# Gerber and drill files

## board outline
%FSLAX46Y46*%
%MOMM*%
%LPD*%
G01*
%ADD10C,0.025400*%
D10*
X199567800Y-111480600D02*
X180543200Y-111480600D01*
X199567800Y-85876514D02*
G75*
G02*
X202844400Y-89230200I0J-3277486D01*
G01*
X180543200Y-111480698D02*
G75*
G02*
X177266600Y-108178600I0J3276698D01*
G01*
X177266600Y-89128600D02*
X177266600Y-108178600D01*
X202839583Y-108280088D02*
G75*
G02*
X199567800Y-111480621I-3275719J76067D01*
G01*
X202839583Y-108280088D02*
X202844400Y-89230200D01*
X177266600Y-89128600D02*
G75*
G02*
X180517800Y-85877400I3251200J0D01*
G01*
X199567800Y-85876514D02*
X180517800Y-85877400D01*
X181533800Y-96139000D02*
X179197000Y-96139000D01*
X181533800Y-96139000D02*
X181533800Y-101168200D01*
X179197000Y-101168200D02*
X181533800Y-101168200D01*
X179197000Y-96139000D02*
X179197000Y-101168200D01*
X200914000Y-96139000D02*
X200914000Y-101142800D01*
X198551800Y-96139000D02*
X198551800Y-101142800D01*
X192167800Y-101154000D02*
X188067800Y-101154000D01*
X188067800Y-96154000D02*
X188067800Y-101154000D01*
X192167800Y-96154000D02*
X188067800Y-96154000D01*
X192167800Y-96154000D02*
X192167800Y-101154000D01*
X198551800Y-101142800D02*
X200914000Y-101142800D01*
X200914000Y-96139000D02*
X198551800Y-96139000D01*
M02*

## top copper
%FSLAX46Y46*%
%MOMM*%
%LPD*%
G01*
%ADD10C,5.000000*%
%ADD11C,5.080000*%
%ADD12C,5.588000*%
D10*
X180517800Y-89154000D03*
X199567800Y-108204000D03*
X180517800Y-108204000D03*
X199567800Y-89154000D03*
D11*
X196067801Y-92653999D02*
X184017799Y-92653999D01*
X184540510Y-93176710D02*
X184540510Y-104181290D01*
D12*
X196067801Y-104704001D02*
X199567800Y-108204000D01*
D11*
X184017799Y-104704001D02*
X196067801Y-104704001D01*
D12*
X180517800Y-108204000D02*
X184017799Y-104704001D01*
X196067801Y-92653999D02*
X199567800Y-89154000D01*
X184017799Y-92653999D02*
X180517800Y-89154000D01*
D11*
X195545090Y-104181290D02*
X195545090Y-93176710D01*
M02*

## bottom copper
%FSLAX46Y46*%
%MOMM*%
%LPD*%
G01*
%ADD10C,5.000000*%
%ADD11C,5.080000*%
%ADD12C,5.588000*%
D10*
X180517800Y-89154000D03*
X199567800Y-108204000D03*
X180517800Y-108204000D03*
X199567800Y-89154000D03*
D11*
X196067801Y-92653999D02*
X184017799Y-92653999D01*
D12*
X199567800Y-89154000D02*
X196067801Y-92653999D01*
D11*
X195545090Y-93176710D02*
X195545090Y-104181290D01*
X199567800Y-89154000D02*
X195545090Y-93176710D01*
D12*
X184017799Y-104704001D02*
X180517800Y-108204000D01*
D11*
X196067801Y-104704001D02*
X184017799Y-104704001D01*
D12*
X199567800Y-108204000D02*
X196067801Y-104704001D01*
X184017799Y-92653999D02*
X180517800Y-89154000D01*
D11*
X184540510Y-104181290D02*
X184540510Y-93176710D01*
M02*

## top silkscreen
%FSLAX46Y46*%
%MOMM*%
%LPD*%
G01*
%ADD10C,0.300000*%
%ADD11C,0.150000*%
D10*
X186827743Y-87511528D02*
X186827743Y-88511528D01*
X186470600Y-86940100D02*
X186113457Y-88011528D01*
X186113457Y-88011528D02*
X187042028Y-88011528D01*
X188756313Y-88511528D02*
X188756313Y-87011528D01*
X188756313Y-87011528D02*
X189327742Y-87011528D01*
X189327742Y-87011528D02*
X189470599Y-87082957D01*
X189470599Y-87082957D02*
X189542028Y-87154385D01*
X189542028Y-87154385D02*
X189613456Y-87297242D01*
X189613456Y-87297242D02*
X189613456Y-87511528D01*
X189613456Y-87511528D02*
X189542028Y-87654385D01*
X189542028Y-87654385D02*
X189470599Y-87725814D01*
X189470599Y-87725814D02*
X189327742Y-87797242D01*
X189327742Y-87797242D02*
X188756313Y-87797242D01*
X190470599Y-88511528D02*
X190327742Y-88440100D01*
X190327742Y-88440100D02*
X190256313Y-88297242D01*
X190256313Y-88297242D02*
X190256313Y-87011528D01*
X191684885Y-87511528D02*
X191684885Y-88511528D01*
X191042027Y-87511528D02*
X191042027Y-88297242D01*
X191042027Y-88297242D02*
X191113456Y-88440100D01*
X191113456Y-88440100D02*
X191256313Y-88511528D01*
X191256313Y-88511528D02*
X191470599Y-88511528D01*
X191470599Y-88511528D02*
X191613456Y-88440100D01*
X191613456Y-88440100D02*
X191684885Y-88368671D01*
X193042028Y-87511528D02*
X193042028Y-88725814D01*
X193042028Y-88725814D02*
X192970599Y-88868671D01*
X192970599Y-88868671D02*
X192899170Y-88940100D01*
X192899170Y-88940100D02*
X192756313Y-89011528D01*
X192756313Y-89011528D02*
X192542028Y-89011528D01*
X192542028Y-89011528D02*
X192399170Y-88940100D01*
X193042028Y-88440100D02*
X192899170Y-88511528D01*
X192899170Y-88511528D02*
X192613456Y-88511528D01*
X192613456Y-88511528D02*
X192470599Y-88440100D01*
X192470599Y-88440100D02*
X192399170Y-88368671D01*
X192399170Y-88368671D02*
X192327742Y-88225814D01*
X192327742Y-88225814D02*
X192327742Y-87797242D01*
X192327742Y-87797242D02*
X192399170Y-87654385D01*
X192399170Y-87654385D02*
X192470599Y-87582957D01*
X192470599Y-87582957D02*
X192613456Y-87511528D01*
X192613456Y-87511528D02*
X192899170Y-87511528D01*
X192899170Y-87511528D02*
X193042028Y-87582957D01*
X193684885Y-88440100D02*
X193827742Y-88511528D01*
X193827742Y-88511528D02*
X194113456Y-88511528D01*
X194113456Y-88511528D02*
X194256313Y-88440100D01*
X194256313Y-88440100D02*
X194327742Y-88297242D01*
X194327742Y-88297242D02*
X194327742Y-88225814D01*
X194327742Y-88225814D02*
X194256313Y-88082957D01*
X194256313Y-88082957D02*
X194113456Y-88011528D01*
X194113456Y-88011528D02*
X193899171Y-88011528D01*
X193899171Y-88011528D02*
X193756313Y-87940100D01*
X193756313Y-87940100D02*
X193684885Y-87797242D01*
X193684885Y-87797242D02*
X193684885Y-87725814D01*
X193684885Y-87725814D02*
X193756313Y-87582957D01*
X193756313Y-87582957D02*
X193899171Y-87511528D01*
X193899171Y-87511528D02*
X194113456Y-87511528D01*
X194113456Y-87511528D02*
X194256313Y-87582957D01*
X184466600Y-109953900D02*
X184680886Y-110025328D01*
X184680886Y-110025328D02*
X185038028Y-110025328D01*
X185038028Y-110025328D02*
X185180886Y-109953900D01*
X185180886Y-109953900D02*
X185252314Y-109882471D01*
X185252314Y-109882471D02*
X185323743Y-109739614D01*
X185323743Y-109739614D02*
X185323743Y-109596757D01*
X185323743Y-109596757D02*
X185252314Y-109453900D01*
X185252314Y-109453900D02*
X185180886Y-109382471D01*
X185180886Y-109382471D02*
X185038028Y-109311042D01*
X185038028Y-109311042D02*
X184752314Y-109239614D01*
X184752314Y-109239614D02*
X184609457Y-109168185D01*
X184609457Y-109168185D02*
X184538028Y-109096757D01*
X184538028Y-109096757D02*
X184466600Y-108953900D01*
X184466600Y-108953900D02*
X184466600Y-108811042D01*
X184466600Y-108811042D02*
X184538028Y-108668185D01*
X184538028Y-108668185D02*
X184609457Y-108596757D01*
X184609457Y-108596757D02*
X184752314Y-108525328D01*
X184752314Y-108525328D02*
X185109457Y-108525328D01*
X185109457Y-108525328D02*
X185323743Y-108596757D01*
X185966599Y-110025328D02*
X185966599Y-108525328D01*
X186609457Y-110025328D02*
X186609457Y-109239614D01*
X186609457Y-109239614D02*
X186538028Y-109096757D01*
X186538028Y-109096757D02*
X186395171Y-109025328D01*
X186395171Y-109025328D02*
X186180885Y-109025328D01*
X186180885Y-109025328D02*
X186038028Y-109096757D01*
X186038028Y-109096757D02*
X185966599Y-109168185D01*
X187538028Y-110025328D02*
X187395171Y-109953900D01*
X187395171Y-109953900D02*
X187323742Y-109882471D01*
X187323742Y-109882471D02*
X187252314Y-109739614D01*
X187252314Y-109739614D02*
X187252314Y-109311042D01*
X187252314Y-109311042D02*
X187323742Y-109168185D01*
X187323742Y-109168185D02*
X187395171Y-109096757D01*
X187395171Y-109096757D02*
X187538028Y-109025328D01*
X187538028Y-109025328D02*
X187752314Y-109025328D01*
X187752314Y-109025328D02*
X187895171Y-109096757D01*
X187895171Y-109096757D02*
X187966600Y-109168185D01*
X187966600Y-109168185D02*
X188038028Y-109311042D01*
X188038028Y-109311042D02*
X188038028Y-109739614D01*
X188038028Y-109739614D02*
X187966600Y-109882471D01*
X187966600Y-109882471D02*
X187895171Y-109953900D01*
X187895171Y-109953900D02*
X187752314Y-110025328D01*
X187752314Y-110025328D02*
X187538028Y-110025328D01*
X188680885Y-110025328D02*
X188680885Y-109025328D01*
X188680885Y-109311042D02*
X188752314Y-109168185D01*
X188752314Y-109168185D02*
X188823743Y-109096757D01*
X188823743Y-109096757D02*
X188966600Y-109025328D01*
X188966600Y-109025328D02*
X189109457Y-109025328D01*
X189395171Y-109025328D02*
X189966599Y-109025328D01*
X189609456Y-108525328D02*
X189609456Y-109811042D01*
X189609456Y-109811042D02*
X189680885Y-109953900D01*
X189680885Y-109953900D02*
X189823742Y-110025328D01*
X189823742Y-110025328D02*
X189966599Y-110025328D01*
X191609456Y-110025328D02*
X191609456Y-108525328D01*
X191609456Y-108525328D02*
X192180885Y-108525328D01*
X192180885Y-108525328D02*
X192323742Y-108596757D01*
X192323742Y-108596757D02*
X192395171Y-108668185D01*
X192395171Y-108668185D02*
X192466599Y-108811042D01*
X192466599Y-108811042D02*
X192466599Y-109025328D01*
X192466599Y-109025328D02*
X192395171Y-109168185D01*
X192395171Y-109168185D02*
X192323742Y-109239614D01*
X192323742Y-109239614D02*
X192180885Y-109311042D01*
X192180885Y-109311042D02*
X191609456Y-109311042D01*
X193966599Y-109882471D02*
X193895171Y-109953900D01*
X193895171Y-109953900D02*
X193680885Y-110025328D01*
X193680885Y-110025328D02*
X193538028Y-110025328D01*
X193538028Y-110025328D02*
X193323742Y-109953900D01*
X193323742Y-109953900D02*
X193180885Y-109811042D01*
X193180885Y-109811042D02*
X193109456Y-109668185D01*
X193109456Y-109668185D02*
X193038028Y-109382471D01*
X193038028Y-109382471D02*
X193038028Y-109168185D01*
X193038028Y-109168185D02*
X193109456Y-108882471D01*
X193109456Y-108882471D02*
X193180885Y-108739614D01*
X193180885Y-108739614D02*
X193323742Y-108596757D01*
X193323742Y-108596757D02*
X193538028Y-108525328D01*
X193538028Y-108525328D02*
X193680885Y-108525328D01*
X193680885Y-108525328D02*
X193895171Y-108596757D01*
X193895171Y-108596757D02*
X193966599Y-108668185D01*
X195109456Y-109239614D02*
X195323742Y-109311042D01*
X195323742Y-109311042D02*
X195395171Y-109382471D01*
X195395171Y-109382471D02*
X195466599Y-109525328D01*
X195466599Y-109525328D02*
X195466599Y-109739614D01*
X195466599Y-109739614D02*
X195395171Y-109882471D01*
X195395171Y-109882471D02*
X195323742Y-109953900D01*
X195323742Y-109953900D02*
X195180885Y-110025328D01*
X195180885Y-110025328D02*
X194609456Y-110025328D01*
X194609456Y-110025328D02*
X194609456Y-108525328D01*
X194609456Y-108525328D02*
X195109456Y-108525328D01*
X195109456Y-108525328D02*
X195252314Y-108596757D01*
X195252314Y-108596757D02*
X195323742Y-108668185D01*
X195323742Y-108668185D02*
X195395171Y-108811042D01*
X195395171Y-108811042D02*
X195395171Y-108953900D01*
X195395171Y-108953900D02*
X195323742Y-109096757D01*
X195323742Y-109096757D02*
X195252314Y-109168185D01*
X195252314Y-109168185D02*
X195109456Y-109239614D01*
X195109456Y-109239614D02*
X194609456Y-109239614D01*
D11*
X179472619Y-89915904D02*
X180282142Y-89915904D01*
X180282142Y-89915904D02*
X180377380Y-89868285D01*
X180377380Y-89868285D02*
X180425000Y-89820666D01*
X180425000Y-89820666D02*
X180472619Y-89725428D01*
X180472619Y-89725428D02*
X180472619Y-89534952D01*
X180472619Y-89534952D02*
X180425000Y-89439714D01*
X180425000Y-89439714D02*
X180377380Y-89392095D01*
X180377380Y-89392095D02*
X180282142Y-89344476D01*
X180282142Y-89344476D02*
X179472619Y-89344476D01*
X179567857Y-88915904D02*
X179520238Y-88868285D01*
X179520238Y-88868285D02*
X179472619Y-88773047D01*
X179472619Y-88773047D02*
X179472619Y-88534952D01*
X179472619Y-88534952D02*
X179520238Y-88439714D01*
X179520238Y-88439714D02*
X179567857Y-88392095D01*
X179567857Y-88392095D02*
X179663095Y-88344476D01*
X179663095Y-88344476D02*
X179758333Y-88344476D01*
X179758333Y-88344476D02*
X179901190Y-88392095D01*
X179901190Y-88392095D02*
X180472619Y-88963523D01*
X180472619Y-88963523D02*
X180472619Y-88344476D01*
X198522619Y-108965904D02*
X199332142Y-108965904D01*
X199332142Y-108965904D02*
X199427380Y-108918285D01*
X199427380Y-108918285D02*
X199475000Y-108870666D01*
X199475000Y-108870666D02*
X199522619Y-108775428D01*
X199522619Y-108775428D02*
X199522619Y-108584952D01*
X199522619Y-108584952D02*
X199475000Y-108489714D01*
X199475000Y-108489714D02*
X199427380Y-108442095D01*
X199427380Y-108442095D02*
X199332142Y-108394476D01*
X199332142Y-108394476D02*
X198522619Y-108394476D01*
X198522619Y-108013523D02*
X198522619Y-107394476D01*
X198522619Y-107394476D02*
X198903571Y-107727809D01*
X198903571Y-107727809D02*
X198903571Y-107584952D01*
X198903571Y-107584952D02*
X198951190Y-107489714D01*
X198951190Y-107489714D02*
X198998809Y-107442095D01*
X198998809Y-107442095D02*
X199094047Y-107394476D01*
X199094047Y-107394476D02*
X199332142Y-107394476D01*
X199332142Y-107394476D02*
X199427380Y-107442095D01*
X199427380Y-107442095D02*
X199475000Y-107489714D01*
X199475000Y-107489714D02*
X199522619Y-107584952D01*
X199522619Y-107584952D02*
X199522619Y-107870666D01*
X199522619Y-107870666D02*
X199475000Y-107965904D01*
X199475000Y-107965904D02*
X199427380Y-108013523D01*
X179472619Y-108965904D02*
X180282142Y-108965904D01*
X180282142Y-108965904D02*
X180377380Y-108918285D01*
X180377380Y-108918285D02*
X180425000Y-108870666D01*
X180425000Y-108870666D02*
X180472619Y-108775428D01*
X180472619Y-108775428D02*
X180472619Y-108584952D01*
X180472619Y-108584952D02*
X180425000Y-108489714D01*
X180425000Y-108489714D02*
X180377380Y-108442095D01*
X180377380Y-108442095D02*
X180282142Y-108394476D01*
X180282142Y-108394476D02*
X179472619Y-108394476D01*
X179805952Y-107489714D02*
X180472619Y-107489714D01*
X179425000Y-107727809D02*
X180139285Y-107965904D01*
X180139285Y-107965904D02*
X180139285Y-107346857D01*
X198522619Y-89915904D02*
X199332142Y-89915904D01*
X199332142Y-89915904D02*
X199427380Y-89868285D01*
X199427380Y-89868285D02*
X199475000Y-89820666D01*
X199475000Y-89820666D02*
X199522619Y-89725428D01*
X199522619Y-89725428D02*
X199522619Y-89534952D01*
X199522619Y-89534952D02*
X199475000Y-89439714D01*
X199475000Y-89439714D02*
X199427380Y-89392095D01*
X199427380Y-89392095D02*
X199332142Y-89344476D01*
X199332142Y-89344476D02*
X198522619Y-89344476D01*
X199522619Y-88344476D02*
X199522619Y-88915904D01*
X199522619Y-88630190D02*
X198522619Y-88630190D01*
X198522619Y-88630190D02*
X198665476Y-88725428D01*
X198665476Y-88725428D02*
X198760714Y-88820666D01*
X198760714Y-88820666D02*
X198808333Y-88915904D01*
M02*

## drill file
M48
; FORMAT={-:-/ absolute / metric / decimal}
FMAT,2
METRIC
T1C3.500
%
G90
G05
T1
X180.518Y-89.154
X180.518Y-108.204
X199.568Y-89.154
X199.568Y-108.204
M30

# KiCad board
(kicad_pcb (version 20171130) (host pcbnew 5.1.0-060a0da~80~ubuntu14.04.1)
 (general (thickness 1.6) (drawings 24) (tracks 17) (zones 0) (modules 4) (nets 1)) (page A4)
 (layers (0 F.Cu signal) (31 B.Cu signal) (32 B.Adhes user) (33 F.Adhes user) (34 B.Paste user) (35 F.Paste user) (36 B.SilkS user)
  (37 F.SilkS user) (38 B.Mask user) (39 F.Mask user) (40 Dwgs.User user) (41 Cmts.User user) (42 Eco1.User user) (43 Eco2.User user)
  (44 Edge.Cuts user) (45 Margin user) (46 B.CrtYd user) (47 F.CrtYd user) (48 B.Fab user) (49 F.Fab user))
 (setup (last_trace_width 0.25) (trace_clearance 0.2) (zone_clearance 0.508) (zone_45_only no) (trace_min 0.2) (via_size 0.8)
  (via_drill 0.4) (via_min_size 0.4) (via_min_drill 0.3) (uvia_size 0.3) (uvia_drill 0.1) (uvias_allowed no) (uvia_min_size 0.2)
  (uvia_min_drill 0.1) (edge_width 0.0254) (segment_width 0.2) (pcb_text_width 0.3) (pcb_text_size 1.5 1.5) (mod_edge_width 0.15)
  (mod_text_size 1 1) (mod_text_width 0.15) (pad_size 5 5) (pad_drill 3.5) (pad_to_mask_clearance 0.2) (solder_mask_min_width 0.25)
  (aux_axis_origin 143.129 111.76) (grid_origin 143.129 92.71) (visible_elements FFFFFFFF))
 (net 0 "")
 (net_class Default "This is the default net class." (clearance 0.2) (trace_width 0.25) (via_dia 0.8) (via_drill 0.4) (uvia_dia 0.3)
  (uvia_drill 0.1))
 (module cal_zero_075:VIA (layer F.Cu) (at 180.5178 89.154 270)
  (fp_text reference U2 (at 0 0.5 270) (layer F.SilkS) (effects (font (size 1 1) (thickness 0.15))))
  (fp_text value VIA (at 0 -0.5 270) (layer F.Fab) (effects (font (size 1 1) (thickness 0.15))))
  (pad 1 thru_hole circle (at 0 0 270) (size 5 5) (drill 3.5) (layers *.Cu *.Mask)))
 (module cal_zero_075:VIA (layer F.Cu) (at 199.5678 108.204 270)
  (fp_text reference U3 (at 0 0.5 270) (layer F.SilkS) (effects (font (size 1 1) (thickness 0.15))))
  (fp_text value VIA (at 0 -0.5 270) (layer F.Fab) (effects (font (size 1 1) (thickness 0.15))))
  (pad 1 thru_hole circle (at 0 0 270) (size 5 5) (drill 3.5) (layers *.Cu *.Mask)))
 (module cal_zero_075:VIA (layer F.Cu) (at 180.5178 108.204 270)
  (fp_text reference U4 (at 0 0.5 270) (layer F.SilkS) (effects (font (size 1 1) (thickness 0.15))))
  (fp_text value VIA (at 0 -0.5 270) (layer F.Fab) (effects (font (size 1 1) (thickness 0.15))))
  (pad 1 thru_hole circle (at 0 0 270) (size 5 5) (drill 3.5) (layers *.Cu *.Mask)))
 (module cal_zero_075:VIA (layer F.Cu) (at 199.5678 89.154 270)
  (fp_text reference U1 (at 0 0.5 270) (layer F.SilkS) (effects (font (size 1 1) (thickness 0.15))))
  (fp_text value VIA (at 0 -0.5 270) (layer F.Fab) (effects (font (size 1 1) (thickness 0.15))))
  (pad 1 thru_hole circle (at 0 0 270) (size 5 5) (drill 3.5) (layers *.Cu *.Mask)))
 (gr_line (start 199.5678 111.4806) (end 180.5432 111.4806) (layer Edge.Cuts) (width 0.0254))
 (gr_arc (start 199.5678 89.154) (end 202.8444 89.2302) (angle -91.33221985) (layer Edge.Cuts) (width 0.0254))
 (gr_arc (start 180.5432 108.204) (end 177.2666 108.1786) (angle -90.44414443) (layer Edge.Cuts) (width 0.0254))
 (gr_line (start 177.2666 89.1286) (end 177.2666 108.1786) (layer Edge.Cuts) (width 0.0254))
 (gr_arc (start 199.563864 108.204021) (end 199.5678 111.480621) (angle -88.60092078) (layer Edge.Cuts) (width 0.0254))
 (gr_line (start 202.839583 108.280088) (end 202.8444 89.2302) (layer Edge.Cuts) (width 0.0254))
 (gr_arc (start 180.5178 89.1286) (end 180.5178 85.8774) (angle -90) (layer Edge.Cuts) (width 0.0254))
 (gr_line (start 199.5678 85.876514) (end 180.5178 85.8774) (layer Edge.Cuts) (width 0.0254))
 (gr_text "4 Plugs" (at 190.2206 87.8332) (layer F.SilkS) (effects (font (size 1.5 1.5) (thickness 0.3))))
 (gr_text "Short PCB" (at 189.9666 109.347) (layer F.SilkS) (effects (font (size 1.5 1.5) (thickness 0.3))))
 (gr_line (start 181.5338 96.139) (end 179.197 96.139) (layer Edge.Cuts) (width 0.0254))
 (gr_line (start 181.5338 96.139) (end 181.5338 101.1682) (layer Edge.Cuts) (width 0.0254))
 (gr_line (start 179.197 101.1682) (end 181.5338 101.1682) (layer Edge.Cuts) (width 0.0254))
 (gr_line (start 179.197 96.139) (end 179.197 101.1682) (layer Edge.Cuts) (width 0.0254))
 (gr_line (start 200.914 96.139) (end 200.914 101.1428) (layer Edge.Cuts) (width 0.0254))
 (gr_line (start 198.5518 96.139) (end 198.5518 101.1428) (layer Edge.Cuts) (width 0.0254))
 (gr_line (start 192.1678 101.154) (end 188.0678 101.154) (layer Edge.Cuts) (width 0.0254))
 (gr_line (start 188.0678 96.154) (end 188.0678 101.154) (layer Edge.Cuts) (width 0.0254))
 (gr_line (start 192.1678 96.154) (end 188.0678 96.154) (layer Edge.Cuts) (width 0.0254))
 (gr_line (start 192.1678 96.154) (end 192.1678 101.154) (layer Edge.Cuts) (width 0.0254))
 (gr_line (start 198.5518 101.1428) (end 200.914 101.1428) (layer Edge.Cuts) (width 0.0254))
 (gr_line (start 200.914 96.139) (end 198.5518 96.139) (layer Edge.Cuts) (width 0.0254))
 (segment (start 196.067801 92.653999) (end 184.017799 92.653999) (width 5.08) (layer F.Cu) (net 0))
 (segment (start 184.54051 93.17671) (end 184.54051 104.18129) (width 5.08) (layer F.Cu) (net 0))
 (segment (start 196.067801 104.704001) (end 199.5678 108.204) (width 5.588) (layer F.Cu) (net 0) (status 20))
 (segment (start 184.017799 104.704001) (end 196.067801 104.704001) (width 5.08) (layer F.Cu) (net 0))
 (segment (start 180.5178 108.204) (end 184.017799 104.704001) (width 5.588) (layer F.Cu) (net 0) (status 10))
 (segment (start 196.067801 92.653999) (end 199.5678 89.154) (width 5.588) (layer F.Cu) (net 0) (status 20))
 (segment (start 196.067801 92.653999) (end 184.017799 92.653999) (width 5.08) (layer B.Cu) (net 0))
 (segment (start 199.5678 89.154) (end 196.067801 92.653999) (width 5.588) (layer B.Cu) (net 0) (status 10))
 (segment (start 195.54509 93.17671) (end 195.54509 104.18129) (width 5.08) (layer B.Cu) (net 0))
 (segment (start 199.5678 89.154) (end 195.54509 93.17671) (width 5.08) (layer B.Cu) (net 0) (status 10))
 (segment (start 184.017799 104.704001) (end 180.5178 108.204) (width 5.588) (layer B.Cu) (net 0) (status 20))
 (segment (start 196.067801 104.704001) (end 184.017799 104.704001) (width 5.08) (layer B.Cu) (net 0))
 (segment (start 199.5678 108.204) (end 196.067801 104.704001) (width 5.588) (layer B.Cu) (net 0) (status 10))
 (segment (start 184.017799 92.653999) (end 180.5178 89.154) (width 5.588) (layer B.Cu) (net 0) (status 20))
 (segment (start 184.54051 104.18129) (end 184.54051 93.17671) (width 5.08) (layer B.Cu) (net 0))
 (segment (start 184.017799 92.653999) (end 180.5178 89.154) (width 5.588) (layer F.Cu) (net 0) (status 20))
 (segment (start 195.54509 104.18129) (end 195.54509 93.17671) (width 5.08) (layer F.Cu) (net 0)))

